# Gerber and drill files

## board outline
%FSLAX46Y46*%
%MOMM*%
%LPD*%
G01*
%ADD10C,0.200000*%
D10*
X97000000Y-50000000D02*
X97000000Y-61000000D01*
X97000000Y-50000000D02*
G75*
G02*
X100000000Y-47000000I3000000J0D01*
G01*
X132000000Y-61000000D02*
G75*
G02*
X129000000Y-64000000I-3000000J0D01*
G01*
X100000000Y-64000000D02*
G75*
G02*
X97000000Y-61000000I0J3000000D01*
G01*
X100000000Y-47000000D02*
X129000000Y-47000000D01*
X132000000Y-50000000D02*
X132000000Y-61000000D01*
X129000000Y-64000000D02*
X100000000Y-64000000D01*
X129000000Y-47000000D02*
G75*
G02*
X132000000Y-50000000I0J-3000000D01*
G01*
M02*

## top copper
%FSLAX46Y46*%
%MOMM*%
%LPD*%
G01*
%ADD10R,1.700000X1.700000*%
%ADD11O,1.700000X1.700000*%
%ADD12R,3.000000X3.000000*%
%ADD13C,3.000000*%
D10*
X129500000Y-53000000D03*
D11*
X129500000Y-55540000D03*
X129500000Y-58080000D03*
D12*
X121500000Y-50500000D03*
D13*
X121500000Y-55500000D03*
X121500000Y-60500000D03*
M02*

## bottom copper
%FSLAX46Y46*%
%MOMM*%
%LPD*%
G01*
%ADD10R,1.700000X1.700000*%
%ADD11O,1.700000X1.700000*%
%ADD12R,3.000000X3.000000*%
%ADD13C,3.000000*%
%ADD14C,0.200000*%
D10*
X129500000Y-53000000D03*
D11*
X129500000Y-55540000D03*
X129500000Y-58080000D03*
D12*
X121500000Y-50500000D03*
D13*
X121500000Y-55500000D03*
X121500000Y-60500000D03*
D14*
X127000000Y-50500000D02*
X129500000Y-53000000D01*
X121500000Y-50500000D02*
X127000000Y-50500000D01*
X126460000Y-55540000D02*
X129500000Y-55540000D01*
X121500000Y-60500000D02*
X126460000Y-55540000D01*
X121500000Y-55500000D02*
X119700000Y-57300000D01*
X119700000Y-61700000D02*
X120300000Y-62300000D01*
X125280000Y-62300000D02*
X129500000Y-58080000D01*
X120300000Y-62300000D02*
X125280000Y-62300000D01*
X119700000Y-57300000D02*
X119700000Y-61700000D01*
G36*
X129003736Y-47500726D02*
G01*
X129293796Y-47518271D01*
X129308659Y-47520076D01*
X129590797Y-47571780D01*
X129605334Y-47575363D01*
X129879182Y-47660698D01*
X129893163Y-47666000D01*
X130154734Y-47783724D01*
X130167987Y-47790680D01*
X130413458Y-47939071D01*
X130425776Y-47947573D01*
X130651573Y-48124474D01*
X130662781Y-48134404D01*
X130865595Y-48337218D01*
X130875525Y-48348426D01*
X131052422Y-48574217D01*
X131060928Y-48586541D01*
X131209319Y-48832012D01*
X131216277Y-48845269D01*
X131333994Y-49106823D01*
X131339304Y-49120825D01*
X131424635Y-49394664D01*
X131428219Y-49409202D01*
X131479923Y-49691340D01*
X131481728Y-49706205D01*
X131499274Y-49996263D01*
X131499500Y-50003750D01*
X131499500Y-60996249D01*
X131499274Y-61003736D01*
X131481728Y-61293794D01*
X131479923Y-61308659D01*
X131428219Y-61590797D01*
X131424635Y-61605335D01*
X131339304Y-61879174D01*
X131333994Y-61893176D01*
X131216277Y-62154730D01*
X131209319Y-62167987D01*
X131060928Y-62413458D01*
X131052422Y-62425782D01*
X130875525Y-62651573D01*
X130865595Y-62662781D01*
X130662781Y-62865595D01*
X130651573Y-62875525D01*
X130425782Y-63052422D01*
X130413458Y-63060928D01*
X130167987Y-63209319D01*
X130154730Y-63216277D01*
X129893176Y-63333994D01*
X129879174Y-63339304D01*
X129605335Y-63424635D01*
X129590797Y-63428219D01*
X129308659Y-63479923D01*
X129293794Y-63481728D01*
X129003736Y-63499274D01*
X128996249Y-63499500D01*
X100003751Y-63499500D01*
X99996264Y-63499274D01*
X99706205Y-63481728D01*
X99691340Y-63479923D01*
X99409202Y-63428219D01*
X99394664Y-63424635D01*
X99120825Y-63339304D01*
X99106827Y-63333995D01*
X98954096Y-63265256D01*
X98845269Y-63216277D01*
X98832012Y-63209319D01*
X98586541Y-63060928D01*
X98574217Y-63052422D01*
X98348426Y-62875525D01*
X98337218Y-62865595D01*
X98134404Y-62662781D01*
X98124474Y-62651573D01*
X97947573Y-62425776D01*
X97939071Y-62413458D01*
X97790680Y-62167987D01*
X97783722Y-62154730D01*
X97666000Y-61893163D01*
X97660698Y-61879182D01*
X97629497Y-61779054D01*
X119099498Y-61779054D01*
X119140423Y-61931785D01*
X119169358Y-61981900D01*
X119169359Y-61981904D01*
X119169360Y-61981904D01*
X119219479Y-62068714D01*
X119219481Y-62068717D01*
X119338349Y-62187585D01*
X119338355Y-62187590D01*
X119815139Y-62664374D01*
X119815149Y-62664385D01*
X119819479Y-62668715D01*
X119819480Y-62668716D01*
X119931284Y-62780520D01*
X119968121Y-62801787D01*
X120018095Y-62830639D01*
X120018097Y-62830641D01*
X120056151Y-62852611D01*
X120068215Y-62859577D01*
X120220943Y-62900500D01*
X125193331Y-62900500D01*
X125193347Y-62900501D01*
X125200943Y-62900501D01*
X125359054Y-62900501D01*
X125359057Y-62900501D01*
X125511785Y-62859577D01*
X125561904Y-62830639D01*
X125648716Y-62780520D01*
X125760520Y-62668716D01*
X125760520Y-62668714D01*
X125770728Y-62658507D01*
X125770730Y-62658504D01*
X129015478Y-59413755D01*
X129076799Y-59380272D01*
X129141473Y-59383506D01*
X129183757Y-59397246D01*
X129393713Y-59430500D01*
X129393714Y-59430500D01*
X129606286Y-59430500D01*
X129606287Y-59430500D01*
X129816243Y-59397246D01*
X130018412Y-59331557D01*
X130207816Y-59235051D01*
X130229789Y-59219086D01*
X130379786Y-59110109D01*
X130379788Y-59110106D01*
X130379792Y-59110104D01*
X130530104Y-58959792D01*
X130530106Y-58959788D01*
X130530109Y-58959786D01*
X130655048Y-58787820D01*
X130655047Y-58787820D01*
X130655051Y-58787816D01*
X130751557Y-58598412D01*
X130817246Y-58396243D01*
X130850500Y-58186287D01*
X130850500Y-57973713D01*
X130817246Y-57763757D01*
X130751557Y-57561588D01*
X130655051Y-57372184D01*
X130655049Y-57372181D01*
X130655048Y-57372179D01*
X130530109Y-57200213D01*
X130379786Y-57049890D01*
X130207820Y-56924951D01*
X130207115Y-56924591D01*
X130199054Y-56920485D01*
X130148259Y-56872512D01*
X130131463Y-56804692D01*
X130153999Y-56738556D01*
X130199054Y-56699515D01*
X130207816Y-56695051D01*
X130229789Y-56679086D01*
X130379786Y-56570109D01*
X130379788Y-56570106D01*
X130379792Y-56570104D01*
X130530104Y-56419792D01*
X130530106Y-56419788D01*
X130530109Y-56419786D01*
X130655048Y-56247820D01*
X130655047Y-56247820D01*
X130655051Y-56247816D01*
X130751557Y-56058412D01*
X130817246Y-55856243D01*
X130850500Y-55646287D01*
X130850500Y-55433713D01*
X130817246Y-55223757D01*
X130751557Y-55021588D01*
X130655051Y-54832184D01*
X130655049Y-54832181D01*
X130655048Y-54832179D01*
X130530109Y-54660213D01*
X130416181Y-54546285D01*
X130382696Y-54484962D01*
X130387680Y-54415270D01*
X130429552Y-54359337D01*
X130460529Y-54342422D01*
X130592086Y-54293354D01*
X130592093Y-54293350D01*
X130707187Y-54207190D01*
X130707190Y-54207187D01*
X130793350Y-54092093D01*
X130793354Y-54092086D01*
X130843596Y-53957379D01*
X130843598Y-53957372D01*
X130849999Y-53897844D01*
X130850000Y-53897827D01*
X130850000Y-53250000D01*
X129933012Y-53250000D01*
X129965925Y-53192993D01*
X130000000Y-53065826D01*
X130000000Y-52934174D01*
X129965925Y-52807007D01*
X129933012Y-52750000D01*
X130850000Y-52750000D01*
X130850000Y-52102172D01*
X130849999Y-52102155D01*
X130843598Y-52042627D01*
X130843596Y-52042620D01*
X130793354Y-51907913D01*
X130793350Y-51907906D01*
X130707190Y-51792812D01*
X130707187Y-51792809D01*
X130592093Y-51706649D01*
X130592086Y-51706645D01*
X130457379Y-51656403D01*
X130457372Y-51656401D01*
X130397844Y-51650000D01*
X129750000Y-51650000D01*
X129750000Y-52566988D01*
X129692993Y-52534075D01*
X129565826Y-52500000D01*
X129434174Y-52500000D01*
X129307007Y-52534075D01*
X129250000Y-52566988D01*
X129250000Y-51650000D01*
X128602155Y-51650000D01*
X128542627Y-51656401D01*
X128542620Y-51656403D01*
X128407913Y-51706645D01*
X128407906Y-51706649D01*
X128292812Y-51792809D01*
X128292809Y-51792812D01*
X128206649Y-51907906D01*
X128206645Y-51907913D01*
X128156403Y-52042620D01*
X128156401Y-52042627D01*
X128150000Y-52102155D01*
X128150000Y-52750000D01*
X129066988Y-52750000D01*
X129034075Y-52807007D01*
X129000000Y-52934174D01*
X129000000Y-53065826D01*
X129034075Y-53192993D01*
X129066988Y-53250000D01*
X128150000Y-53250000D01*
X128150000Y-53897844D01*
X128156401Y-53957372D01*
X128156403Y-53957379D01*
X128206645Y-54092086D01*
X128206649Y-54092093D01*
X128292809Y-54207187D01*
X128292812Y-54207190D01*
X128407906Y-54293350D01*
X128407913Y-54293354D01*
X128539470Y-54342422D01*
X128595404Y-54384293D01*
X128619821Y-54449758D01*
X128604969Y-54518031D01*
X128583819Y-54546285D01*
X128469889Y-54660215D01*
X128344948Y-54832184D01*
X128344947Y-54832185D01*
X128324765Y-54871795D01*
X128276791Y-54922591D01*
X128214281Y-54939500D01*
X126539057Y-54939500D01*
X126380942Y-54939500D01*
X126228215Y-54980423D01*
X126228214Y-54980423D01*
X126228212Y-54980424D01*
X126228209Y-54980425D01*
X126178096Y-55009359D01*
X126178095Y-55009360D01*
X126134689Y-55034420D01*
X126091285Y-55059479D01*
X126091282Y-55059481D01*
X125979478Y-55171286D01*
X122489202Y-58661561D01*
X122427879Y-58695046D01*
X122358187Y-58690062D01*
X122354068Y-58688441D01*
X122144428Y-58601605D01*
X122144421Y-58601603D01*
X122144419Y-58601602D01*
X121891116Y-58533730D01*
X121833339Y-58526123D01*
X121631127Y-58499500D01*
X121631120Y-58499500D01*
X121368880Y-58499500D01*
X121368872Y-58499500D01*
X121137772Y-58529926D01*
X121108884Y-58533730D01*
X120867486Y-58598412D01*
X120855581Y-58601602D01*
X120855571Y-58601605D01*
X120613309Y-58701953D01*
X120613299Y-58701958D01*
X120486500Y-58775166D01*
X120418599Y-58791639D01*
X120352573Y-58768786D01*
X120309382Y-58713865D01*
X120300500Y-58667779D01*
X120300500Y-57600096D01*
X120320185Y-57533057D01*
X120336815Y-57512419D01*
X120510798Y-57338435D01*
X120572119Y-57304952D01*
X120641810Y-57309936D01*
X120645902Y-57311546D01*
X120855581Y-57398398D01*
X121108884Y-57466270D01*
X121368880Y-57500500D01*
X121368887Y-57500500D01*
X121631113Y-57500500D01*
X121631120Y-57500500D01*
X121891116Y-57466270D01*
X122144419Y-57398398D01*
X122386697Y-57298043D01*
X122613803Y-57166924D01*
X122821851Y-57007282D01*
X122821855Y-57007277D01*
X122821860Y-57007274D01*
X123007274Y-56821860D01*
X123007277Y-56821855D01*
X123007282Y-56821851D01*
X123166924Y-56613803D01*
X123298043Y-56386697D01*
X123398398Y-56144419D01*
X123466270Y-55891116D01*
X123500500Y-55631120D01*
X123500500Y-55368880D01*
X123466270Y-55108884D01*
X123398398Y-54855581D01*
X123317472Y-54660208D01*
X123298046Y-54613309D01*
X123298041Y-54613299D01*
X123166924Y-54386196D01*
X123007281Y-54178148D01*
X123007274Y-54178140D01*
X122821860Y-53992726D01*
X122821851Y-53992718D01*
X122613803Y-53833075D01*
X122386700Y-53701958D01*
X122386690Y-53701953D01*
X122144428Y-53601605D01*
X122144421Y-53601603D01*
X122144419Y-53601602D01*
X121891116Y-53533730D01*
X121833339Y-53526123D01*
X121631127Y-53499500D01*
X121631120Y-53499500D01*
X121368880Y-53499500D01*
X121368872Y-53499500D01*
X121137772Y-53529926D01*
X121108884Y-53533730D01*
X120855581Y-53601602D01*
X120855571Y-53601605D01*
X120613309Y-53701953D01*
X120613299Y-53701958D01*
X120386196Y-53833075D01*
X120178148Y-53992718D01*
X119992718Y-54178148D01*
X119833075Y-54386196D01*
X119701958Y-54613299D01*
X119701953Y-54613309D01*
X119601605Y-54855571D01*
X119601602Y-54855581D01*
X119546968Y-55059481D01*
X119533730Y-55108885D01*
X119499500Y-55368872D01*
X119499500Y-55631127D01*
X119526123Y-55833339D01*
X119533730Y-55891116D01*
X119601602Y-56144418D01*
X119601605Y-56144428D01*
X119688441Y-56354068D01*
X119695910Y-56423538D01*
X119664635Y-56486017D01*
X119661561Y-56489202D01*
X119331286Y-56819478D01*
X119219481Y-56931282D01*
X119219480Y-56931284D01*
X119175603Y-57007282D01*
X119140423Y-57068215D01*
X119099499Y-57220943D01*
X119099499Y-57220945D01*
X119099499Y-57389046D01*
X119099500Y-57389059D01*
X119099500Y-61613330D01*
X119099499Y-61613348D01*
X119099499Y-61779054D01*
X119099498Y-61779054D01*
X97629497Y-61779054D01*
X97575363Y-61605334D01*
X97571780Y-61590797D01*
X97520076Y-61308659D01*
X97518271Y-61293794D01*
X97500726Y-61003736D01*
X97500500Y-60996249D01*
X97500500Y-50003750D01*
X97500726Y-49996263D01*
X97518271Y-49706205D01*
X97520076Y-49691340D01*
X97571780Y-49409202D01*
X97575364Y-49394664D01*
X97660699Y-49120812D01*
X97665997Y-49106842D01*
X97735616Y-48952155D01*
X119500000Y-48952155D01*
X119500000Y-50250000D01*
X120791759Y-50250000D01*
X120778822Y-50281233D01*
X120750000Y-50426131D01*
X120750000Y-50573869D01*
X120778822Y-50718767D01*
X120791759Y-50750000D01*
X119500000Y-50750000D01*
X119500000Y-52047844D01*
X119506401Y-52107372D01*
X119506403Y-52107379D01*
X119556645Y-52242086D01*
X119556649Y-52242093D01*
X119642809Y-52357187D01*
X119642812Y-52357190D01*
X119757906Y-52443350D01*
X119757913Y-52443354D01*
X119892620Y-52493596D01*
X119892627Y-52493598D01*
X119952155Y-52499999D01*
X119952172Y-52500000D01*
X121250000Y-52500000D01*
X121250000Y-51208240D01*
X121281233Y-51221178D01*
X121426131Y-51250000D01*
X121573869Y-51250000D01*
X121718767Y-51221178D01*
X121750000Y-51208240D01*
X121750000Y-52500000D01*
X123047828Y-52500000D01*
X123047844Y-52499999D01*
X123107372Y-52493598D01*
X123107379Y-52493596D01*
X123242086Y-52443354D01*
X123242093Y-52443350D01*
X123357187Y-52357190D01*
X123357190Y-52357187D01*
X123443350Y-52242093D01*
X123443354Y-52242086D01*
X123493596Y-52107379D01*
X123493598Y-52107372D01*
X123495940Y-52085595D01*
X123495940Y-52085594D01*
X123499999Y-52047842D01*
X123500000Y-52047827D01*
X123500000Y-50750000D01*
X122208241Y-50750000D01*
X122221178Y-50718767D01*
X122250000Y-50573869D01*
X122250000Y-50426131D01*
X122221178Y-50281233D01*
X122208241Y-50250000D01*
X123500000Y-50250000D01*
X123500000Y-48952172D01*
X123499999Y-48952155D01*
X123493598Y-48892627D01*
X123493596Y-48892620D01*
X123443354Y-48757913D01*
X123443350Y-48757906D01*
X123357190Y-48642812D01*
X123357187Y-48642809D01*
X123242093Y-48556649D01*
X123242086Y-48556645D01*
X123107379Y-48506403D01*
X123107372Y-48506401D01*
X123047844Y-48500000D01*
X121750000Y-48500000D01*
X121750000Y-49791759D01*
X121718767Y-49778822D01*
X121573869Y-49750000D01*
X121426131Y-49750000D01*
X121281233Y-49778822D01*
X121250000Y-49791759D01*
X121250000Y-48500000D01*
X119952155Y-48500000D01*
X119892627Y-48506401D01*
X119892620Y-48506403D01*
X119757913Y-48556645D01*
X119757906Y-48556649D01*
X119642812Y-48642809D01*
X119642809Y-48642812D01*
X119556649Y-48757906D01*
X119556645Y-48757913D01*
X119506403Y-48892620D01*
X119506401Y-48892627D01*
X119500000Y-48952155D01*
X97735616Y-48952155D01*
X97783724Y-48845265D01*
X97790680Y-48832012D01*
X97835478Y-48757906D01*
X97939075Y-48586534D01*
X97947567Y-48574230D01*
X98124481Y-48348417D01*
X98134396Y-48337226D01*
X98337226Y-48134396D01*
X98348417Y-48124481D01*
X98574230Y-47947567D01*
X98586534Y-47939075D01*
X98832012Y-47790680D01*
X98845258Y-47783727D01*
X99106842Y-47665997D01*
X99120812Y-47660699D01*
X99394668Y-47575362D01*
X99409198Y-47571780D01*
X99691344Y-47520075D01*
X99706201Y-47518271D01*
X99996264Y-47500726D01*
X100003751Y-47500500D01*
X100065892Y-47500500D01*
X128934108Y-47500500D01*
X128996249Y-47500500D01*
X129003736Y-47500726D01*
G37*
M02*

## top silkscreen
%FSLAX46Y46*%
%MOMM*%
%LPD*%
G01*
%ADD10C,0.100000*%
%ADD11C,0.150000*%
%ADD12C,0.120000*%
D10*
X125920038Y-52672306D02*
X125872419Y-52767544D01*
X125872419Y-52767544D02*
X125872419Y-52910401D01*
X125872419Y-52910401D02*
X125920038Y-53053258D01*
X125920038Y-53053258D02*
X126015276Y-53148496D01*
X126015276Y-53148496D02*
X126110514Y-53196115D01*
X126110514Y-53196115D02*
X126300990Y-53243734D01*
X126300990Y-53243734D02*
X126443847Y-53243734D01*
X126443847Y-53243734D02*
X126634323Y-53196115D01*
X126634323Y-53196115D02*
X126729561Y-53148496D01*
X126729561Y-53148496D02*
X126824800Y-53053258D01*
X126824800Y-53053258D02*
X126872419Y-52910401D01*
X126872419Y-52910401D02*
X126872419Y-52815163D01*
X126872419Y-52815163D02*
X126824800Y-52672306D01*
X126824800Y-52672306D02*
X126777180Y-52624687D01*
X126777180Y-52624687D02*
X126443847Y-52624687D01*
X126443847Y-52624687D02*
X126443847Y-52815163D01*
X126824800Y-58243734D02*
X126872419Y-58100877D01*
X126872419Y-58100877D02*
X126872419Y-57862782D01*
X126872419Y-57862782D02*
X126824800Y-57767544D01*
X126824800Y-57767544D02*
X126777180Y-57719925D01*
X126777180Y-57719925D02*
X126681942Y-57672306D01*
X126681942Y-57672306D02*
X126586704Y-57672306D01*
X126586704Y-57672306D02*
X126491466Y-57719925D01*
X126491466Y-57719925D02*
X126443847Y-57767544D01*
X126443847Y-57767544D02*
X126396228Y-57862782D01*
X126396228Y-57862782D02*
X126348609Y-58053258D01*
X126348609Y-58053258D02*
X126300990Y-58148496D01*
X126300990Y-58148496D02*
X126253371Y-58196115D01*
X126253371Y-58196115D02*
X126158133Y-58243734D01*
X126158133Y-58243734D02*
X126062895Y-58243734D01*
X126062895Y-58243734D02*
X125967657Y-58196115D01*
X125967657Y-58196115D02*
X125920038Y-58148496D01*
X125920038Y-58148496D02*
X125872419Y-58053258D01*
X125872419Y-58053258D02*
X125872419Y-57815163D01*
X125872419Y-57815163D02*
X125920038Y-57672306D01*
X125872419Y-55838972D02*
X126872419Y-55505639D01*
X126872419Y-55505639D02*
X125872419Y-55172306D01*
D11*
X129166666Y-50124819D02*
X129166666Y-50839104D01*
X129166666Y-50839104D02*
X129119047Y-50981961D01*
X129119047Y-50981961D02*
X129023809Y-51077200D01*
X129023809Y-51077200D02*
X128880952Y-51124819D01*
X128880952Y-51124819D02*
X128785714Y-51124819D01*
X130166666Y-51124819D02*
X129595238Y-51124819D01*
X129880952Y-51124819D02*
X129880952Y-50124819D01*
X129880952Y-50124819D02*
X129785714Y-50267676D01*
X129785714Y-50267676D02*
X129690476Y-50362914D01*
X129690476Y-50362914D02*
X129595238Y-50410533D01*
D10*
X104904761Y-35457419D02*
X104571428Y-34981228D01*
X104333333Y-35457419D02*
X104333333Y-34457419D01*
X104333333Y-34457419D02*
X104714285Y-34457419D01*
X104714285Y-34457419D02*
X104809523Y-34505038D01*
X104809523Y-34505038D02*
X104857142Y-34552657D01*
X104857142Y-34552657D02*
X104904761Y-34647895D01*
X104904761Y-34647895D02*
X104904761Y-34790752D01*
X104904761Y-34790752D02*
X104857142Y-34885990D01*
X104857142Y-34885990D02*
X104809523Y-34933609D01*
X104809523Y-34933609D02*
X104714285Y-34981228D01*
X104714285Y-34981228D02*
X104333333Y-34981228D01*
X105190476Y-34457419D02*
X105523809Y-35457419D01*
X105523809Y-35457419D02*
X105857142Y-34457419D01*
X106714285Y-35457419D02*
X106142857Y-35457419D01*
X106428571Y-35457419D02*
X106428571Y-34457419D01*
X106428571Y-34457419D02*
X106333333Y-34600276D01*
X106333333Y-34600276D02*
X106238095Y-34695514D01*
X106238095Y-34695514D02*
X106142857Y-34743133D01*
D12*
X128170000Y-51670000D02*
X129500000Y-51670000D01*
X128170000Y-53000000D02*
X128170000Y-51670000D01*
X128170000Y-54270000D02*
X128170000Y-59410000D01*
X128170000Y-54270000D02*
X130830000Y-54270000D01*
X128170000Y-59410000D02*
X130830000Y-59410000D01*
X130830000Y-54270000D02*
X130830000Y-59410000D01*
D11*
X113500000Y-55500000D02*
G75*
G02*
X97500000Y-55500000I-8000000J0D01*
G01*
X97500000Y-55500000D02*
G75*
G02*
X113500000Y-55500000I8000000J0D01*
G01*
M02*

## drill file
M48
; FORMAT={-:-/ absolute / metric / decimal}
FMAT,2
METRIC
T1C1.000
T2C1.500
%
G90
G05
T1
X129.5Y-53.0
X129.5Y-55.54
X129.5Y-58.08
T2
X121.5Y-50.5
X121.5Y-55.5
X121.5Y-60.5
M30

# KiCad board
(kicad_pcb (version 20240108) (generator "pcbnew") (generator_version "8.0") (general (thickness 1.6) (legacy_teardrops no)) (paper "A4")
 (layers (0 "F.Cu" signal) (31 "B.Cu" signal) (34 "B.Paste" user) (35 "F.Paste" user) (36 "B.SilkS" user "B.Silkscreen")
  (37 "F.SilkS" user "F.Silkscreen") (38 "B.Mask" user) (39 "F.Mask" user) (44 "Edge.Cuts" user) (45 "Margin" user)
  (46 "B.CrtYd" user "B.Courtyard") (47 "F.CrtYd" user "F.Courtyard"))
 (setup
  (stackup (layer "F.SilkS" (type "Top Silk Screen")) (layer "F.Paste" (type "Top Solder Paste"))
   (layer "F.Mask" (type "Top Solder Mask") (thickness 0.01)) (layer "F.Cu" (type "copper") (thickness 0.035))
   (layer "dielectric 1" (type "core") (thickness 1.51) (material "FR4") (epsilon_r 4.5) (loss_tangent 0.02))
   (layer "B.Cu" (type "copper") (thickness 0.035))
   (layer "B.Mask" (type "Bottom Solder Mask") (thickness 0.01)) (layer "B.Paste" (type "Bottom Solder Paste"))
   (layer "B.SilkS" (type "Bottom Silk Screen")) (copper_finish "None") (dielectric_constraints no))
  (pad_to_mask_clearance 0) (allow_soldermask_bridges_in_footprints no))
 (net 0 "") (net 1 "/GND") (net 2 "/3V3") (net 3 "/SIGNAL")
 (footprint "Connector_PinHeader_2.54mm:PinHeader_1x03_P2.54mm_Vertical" (layer "F.Cu") (at 129.5 53)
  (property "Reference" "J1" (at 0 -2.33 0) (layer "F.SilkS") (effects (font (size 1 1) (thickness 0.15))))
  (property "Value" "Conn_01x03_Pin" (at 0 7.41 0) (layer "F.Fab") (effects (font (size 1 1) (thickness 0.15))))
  (fp_line (start -1.33 -1.33) (end 0 -1.33) (stroke (width 0.12) (type solid)) (layer "F.SilkS"))
  (fp_line (start -1.33 0) (end -1.33 -1.33) (stroke (width 0.12) (type solid)) (layer "F.SilkS"))
  (fp_line (start -1.33 1.27) (end -1.33 6.41) (stroke (width 0.12) (type solid)) (layer "F.SilkS"))
  (fp_line (start -1.33 1.27) (end 1.33 1.27) (stroke (width 0.12) (type solid)) (layer "F.SilkS"))
  (fp_line (start -1.33 6.41) (end 1.33 6.41) (stroke (width 0.12) (type solid)) (layer "F.SilkS"))
  (fp_line (start 1.33 1.27) (end 1.33 6.41) (stroke (width 0.12) (type solid)) (layer "F.SilkS"))
  (pad "1" thru_hole rect (at 0 0) (size 1.7 1.7) (drill 1) (layers "*.Cu" "*.Mask") (remove_unused_layers no) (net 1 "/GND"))
  (pad "2" thru_hole oval (at 0 2.54) (size 1.7 1.7) (drill 1) (layers "*.Cu" "*.Mask") (remove_unused_layers no) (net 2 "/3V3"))
  (pad "3" thru_hole oval (at 0 5.08) (size 1.7 1.7) (drill 1) (layers "*.Cu" "*.Mask") (remove_unused_layers no) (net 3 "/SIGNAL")))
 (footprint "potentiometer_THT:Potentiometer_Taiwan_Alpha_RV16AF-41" (layer "F.Cu") (at 105.5 55.5)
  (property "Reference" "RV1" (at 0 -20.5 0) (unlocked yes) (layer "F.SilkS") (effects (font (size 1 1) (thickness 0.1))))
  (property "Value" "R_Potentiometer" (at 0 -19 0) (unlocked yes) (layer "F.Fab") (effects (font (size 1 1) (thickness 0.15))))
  (fp_circle (center 0 0) (end 8 0) (stroke (width 0.15) (type default)) (fill none) (layer "F.SilkS"))
  (pad "1" thru_hole rect (at 16 -5) (size 3 3) (drill 1.5) (layers "*.Cu" "*.Mask") (remove_unused_layers no) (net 1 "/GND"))
  (pad "2" thru_hole circle (at 16 0) (size 3 3) (drill 1.5) (layers "*.Cu" "*.Mask") (remove_unused_layers no) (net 3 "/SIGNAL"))
  (pad "3" thru_hole circle (at 16 5) (size 3 3) (drill 1.5) (layers "*.Cu" "*.Mask") (remove_unused_layers no) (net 2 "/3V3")))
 (gr_line (start 97 50) (end 97 61) (locked yes) (stroke (width 0.2) (type default)) (layer "Edge.Cuts"))
 (gr_arc (start 97 50) (mid 97.87868 47.87868) (end 100 47) (locked yes) (stroke (width 0.2) (type default)) (layer "Edge.Cuts"))
 (gr_arc (start 132 61) (mid 131.12132 63.12132) (end 129 64) (locked yes) (stroke (width 0.2) (type default)) (layer "Edge.Cuts"))
 (gr_arc (start 100 64) (mid 97.87868 63.12132) (end 97 61) (locked yes) (stroke (width 0.2) (type default)) (layer "Edge.Cuts"))
 (gr_line (start 100 47) (end 129 47) (locked yes) (stroke (width 0.2) (type default)) (layer "Edge.Cuts"))
 (gr_line (start 132 50) (end 132 61) (locked yes) (stroke (width 0.2) (type default)) (layer "Edge.Cuts"))
 (gr_line (start 129 64) (end 100 64) (locked yes) (stroke (width 0.2) (type default)) (layer "Edge.Cuts"))
 (gr_arc (start 129 47) (mid 131.12132 47.87868) (end 132 50) (locked yes) (stroke (width 0.2) (type default)) (layer "Edge.Cuts"))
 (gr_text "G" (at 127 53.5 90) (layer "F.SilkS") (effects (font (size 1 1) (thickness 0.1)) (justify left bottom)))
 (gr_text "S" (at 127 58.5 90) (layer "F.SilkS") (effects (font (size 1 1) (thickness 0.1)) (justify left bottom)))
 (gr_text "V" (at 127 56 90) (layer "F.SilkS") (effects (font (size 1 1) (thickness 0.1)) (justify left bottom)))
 (segment (start 127 50.5) (end 129.5 53) (width 0.2) (layer "B.Cu") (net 1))
 (segment (start 121.5 50.5) (end 127 50.5) (width 0.2) (layer "B.Cu") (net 1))
 (segment (start 126.46 55.54) (end 129.5 55.54) (width 0.2) (layer "B.Cu") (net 2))
 (segment (start 121.5 60.5) (end 126.46 55.54) (width 0.2) (layer "B.Cu") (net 2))
 (segment (start 121.5 55.5) (end 119.7 57.3) (width 0.2) (layer "B.Cu") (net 3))
 (segment (start 119.7 61.7) (end 120.3 62.3) (width 0.2) (layer "B.Cu") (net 3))
 (segment (start 125.28 62.3) (end 129.5 58.08) (width 0.2) (layer "B.Cu") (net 3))
 (segment (start 120.3 62.3) (end 125.28 62.3) (width 0.2) (layer "B.Cu") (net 3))
 (segment (start 119.7 57.3) (end 119.7 61.7) (width 0.2) (layer "B.Cu") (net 3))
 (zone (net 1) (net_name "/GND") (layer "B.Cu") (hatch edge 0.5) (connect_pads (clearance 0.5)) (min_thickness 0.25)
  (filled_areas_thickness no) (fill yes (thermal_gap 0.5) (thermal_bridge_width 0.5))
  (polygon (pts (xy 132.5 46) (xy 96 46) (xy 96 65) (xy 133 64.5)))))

